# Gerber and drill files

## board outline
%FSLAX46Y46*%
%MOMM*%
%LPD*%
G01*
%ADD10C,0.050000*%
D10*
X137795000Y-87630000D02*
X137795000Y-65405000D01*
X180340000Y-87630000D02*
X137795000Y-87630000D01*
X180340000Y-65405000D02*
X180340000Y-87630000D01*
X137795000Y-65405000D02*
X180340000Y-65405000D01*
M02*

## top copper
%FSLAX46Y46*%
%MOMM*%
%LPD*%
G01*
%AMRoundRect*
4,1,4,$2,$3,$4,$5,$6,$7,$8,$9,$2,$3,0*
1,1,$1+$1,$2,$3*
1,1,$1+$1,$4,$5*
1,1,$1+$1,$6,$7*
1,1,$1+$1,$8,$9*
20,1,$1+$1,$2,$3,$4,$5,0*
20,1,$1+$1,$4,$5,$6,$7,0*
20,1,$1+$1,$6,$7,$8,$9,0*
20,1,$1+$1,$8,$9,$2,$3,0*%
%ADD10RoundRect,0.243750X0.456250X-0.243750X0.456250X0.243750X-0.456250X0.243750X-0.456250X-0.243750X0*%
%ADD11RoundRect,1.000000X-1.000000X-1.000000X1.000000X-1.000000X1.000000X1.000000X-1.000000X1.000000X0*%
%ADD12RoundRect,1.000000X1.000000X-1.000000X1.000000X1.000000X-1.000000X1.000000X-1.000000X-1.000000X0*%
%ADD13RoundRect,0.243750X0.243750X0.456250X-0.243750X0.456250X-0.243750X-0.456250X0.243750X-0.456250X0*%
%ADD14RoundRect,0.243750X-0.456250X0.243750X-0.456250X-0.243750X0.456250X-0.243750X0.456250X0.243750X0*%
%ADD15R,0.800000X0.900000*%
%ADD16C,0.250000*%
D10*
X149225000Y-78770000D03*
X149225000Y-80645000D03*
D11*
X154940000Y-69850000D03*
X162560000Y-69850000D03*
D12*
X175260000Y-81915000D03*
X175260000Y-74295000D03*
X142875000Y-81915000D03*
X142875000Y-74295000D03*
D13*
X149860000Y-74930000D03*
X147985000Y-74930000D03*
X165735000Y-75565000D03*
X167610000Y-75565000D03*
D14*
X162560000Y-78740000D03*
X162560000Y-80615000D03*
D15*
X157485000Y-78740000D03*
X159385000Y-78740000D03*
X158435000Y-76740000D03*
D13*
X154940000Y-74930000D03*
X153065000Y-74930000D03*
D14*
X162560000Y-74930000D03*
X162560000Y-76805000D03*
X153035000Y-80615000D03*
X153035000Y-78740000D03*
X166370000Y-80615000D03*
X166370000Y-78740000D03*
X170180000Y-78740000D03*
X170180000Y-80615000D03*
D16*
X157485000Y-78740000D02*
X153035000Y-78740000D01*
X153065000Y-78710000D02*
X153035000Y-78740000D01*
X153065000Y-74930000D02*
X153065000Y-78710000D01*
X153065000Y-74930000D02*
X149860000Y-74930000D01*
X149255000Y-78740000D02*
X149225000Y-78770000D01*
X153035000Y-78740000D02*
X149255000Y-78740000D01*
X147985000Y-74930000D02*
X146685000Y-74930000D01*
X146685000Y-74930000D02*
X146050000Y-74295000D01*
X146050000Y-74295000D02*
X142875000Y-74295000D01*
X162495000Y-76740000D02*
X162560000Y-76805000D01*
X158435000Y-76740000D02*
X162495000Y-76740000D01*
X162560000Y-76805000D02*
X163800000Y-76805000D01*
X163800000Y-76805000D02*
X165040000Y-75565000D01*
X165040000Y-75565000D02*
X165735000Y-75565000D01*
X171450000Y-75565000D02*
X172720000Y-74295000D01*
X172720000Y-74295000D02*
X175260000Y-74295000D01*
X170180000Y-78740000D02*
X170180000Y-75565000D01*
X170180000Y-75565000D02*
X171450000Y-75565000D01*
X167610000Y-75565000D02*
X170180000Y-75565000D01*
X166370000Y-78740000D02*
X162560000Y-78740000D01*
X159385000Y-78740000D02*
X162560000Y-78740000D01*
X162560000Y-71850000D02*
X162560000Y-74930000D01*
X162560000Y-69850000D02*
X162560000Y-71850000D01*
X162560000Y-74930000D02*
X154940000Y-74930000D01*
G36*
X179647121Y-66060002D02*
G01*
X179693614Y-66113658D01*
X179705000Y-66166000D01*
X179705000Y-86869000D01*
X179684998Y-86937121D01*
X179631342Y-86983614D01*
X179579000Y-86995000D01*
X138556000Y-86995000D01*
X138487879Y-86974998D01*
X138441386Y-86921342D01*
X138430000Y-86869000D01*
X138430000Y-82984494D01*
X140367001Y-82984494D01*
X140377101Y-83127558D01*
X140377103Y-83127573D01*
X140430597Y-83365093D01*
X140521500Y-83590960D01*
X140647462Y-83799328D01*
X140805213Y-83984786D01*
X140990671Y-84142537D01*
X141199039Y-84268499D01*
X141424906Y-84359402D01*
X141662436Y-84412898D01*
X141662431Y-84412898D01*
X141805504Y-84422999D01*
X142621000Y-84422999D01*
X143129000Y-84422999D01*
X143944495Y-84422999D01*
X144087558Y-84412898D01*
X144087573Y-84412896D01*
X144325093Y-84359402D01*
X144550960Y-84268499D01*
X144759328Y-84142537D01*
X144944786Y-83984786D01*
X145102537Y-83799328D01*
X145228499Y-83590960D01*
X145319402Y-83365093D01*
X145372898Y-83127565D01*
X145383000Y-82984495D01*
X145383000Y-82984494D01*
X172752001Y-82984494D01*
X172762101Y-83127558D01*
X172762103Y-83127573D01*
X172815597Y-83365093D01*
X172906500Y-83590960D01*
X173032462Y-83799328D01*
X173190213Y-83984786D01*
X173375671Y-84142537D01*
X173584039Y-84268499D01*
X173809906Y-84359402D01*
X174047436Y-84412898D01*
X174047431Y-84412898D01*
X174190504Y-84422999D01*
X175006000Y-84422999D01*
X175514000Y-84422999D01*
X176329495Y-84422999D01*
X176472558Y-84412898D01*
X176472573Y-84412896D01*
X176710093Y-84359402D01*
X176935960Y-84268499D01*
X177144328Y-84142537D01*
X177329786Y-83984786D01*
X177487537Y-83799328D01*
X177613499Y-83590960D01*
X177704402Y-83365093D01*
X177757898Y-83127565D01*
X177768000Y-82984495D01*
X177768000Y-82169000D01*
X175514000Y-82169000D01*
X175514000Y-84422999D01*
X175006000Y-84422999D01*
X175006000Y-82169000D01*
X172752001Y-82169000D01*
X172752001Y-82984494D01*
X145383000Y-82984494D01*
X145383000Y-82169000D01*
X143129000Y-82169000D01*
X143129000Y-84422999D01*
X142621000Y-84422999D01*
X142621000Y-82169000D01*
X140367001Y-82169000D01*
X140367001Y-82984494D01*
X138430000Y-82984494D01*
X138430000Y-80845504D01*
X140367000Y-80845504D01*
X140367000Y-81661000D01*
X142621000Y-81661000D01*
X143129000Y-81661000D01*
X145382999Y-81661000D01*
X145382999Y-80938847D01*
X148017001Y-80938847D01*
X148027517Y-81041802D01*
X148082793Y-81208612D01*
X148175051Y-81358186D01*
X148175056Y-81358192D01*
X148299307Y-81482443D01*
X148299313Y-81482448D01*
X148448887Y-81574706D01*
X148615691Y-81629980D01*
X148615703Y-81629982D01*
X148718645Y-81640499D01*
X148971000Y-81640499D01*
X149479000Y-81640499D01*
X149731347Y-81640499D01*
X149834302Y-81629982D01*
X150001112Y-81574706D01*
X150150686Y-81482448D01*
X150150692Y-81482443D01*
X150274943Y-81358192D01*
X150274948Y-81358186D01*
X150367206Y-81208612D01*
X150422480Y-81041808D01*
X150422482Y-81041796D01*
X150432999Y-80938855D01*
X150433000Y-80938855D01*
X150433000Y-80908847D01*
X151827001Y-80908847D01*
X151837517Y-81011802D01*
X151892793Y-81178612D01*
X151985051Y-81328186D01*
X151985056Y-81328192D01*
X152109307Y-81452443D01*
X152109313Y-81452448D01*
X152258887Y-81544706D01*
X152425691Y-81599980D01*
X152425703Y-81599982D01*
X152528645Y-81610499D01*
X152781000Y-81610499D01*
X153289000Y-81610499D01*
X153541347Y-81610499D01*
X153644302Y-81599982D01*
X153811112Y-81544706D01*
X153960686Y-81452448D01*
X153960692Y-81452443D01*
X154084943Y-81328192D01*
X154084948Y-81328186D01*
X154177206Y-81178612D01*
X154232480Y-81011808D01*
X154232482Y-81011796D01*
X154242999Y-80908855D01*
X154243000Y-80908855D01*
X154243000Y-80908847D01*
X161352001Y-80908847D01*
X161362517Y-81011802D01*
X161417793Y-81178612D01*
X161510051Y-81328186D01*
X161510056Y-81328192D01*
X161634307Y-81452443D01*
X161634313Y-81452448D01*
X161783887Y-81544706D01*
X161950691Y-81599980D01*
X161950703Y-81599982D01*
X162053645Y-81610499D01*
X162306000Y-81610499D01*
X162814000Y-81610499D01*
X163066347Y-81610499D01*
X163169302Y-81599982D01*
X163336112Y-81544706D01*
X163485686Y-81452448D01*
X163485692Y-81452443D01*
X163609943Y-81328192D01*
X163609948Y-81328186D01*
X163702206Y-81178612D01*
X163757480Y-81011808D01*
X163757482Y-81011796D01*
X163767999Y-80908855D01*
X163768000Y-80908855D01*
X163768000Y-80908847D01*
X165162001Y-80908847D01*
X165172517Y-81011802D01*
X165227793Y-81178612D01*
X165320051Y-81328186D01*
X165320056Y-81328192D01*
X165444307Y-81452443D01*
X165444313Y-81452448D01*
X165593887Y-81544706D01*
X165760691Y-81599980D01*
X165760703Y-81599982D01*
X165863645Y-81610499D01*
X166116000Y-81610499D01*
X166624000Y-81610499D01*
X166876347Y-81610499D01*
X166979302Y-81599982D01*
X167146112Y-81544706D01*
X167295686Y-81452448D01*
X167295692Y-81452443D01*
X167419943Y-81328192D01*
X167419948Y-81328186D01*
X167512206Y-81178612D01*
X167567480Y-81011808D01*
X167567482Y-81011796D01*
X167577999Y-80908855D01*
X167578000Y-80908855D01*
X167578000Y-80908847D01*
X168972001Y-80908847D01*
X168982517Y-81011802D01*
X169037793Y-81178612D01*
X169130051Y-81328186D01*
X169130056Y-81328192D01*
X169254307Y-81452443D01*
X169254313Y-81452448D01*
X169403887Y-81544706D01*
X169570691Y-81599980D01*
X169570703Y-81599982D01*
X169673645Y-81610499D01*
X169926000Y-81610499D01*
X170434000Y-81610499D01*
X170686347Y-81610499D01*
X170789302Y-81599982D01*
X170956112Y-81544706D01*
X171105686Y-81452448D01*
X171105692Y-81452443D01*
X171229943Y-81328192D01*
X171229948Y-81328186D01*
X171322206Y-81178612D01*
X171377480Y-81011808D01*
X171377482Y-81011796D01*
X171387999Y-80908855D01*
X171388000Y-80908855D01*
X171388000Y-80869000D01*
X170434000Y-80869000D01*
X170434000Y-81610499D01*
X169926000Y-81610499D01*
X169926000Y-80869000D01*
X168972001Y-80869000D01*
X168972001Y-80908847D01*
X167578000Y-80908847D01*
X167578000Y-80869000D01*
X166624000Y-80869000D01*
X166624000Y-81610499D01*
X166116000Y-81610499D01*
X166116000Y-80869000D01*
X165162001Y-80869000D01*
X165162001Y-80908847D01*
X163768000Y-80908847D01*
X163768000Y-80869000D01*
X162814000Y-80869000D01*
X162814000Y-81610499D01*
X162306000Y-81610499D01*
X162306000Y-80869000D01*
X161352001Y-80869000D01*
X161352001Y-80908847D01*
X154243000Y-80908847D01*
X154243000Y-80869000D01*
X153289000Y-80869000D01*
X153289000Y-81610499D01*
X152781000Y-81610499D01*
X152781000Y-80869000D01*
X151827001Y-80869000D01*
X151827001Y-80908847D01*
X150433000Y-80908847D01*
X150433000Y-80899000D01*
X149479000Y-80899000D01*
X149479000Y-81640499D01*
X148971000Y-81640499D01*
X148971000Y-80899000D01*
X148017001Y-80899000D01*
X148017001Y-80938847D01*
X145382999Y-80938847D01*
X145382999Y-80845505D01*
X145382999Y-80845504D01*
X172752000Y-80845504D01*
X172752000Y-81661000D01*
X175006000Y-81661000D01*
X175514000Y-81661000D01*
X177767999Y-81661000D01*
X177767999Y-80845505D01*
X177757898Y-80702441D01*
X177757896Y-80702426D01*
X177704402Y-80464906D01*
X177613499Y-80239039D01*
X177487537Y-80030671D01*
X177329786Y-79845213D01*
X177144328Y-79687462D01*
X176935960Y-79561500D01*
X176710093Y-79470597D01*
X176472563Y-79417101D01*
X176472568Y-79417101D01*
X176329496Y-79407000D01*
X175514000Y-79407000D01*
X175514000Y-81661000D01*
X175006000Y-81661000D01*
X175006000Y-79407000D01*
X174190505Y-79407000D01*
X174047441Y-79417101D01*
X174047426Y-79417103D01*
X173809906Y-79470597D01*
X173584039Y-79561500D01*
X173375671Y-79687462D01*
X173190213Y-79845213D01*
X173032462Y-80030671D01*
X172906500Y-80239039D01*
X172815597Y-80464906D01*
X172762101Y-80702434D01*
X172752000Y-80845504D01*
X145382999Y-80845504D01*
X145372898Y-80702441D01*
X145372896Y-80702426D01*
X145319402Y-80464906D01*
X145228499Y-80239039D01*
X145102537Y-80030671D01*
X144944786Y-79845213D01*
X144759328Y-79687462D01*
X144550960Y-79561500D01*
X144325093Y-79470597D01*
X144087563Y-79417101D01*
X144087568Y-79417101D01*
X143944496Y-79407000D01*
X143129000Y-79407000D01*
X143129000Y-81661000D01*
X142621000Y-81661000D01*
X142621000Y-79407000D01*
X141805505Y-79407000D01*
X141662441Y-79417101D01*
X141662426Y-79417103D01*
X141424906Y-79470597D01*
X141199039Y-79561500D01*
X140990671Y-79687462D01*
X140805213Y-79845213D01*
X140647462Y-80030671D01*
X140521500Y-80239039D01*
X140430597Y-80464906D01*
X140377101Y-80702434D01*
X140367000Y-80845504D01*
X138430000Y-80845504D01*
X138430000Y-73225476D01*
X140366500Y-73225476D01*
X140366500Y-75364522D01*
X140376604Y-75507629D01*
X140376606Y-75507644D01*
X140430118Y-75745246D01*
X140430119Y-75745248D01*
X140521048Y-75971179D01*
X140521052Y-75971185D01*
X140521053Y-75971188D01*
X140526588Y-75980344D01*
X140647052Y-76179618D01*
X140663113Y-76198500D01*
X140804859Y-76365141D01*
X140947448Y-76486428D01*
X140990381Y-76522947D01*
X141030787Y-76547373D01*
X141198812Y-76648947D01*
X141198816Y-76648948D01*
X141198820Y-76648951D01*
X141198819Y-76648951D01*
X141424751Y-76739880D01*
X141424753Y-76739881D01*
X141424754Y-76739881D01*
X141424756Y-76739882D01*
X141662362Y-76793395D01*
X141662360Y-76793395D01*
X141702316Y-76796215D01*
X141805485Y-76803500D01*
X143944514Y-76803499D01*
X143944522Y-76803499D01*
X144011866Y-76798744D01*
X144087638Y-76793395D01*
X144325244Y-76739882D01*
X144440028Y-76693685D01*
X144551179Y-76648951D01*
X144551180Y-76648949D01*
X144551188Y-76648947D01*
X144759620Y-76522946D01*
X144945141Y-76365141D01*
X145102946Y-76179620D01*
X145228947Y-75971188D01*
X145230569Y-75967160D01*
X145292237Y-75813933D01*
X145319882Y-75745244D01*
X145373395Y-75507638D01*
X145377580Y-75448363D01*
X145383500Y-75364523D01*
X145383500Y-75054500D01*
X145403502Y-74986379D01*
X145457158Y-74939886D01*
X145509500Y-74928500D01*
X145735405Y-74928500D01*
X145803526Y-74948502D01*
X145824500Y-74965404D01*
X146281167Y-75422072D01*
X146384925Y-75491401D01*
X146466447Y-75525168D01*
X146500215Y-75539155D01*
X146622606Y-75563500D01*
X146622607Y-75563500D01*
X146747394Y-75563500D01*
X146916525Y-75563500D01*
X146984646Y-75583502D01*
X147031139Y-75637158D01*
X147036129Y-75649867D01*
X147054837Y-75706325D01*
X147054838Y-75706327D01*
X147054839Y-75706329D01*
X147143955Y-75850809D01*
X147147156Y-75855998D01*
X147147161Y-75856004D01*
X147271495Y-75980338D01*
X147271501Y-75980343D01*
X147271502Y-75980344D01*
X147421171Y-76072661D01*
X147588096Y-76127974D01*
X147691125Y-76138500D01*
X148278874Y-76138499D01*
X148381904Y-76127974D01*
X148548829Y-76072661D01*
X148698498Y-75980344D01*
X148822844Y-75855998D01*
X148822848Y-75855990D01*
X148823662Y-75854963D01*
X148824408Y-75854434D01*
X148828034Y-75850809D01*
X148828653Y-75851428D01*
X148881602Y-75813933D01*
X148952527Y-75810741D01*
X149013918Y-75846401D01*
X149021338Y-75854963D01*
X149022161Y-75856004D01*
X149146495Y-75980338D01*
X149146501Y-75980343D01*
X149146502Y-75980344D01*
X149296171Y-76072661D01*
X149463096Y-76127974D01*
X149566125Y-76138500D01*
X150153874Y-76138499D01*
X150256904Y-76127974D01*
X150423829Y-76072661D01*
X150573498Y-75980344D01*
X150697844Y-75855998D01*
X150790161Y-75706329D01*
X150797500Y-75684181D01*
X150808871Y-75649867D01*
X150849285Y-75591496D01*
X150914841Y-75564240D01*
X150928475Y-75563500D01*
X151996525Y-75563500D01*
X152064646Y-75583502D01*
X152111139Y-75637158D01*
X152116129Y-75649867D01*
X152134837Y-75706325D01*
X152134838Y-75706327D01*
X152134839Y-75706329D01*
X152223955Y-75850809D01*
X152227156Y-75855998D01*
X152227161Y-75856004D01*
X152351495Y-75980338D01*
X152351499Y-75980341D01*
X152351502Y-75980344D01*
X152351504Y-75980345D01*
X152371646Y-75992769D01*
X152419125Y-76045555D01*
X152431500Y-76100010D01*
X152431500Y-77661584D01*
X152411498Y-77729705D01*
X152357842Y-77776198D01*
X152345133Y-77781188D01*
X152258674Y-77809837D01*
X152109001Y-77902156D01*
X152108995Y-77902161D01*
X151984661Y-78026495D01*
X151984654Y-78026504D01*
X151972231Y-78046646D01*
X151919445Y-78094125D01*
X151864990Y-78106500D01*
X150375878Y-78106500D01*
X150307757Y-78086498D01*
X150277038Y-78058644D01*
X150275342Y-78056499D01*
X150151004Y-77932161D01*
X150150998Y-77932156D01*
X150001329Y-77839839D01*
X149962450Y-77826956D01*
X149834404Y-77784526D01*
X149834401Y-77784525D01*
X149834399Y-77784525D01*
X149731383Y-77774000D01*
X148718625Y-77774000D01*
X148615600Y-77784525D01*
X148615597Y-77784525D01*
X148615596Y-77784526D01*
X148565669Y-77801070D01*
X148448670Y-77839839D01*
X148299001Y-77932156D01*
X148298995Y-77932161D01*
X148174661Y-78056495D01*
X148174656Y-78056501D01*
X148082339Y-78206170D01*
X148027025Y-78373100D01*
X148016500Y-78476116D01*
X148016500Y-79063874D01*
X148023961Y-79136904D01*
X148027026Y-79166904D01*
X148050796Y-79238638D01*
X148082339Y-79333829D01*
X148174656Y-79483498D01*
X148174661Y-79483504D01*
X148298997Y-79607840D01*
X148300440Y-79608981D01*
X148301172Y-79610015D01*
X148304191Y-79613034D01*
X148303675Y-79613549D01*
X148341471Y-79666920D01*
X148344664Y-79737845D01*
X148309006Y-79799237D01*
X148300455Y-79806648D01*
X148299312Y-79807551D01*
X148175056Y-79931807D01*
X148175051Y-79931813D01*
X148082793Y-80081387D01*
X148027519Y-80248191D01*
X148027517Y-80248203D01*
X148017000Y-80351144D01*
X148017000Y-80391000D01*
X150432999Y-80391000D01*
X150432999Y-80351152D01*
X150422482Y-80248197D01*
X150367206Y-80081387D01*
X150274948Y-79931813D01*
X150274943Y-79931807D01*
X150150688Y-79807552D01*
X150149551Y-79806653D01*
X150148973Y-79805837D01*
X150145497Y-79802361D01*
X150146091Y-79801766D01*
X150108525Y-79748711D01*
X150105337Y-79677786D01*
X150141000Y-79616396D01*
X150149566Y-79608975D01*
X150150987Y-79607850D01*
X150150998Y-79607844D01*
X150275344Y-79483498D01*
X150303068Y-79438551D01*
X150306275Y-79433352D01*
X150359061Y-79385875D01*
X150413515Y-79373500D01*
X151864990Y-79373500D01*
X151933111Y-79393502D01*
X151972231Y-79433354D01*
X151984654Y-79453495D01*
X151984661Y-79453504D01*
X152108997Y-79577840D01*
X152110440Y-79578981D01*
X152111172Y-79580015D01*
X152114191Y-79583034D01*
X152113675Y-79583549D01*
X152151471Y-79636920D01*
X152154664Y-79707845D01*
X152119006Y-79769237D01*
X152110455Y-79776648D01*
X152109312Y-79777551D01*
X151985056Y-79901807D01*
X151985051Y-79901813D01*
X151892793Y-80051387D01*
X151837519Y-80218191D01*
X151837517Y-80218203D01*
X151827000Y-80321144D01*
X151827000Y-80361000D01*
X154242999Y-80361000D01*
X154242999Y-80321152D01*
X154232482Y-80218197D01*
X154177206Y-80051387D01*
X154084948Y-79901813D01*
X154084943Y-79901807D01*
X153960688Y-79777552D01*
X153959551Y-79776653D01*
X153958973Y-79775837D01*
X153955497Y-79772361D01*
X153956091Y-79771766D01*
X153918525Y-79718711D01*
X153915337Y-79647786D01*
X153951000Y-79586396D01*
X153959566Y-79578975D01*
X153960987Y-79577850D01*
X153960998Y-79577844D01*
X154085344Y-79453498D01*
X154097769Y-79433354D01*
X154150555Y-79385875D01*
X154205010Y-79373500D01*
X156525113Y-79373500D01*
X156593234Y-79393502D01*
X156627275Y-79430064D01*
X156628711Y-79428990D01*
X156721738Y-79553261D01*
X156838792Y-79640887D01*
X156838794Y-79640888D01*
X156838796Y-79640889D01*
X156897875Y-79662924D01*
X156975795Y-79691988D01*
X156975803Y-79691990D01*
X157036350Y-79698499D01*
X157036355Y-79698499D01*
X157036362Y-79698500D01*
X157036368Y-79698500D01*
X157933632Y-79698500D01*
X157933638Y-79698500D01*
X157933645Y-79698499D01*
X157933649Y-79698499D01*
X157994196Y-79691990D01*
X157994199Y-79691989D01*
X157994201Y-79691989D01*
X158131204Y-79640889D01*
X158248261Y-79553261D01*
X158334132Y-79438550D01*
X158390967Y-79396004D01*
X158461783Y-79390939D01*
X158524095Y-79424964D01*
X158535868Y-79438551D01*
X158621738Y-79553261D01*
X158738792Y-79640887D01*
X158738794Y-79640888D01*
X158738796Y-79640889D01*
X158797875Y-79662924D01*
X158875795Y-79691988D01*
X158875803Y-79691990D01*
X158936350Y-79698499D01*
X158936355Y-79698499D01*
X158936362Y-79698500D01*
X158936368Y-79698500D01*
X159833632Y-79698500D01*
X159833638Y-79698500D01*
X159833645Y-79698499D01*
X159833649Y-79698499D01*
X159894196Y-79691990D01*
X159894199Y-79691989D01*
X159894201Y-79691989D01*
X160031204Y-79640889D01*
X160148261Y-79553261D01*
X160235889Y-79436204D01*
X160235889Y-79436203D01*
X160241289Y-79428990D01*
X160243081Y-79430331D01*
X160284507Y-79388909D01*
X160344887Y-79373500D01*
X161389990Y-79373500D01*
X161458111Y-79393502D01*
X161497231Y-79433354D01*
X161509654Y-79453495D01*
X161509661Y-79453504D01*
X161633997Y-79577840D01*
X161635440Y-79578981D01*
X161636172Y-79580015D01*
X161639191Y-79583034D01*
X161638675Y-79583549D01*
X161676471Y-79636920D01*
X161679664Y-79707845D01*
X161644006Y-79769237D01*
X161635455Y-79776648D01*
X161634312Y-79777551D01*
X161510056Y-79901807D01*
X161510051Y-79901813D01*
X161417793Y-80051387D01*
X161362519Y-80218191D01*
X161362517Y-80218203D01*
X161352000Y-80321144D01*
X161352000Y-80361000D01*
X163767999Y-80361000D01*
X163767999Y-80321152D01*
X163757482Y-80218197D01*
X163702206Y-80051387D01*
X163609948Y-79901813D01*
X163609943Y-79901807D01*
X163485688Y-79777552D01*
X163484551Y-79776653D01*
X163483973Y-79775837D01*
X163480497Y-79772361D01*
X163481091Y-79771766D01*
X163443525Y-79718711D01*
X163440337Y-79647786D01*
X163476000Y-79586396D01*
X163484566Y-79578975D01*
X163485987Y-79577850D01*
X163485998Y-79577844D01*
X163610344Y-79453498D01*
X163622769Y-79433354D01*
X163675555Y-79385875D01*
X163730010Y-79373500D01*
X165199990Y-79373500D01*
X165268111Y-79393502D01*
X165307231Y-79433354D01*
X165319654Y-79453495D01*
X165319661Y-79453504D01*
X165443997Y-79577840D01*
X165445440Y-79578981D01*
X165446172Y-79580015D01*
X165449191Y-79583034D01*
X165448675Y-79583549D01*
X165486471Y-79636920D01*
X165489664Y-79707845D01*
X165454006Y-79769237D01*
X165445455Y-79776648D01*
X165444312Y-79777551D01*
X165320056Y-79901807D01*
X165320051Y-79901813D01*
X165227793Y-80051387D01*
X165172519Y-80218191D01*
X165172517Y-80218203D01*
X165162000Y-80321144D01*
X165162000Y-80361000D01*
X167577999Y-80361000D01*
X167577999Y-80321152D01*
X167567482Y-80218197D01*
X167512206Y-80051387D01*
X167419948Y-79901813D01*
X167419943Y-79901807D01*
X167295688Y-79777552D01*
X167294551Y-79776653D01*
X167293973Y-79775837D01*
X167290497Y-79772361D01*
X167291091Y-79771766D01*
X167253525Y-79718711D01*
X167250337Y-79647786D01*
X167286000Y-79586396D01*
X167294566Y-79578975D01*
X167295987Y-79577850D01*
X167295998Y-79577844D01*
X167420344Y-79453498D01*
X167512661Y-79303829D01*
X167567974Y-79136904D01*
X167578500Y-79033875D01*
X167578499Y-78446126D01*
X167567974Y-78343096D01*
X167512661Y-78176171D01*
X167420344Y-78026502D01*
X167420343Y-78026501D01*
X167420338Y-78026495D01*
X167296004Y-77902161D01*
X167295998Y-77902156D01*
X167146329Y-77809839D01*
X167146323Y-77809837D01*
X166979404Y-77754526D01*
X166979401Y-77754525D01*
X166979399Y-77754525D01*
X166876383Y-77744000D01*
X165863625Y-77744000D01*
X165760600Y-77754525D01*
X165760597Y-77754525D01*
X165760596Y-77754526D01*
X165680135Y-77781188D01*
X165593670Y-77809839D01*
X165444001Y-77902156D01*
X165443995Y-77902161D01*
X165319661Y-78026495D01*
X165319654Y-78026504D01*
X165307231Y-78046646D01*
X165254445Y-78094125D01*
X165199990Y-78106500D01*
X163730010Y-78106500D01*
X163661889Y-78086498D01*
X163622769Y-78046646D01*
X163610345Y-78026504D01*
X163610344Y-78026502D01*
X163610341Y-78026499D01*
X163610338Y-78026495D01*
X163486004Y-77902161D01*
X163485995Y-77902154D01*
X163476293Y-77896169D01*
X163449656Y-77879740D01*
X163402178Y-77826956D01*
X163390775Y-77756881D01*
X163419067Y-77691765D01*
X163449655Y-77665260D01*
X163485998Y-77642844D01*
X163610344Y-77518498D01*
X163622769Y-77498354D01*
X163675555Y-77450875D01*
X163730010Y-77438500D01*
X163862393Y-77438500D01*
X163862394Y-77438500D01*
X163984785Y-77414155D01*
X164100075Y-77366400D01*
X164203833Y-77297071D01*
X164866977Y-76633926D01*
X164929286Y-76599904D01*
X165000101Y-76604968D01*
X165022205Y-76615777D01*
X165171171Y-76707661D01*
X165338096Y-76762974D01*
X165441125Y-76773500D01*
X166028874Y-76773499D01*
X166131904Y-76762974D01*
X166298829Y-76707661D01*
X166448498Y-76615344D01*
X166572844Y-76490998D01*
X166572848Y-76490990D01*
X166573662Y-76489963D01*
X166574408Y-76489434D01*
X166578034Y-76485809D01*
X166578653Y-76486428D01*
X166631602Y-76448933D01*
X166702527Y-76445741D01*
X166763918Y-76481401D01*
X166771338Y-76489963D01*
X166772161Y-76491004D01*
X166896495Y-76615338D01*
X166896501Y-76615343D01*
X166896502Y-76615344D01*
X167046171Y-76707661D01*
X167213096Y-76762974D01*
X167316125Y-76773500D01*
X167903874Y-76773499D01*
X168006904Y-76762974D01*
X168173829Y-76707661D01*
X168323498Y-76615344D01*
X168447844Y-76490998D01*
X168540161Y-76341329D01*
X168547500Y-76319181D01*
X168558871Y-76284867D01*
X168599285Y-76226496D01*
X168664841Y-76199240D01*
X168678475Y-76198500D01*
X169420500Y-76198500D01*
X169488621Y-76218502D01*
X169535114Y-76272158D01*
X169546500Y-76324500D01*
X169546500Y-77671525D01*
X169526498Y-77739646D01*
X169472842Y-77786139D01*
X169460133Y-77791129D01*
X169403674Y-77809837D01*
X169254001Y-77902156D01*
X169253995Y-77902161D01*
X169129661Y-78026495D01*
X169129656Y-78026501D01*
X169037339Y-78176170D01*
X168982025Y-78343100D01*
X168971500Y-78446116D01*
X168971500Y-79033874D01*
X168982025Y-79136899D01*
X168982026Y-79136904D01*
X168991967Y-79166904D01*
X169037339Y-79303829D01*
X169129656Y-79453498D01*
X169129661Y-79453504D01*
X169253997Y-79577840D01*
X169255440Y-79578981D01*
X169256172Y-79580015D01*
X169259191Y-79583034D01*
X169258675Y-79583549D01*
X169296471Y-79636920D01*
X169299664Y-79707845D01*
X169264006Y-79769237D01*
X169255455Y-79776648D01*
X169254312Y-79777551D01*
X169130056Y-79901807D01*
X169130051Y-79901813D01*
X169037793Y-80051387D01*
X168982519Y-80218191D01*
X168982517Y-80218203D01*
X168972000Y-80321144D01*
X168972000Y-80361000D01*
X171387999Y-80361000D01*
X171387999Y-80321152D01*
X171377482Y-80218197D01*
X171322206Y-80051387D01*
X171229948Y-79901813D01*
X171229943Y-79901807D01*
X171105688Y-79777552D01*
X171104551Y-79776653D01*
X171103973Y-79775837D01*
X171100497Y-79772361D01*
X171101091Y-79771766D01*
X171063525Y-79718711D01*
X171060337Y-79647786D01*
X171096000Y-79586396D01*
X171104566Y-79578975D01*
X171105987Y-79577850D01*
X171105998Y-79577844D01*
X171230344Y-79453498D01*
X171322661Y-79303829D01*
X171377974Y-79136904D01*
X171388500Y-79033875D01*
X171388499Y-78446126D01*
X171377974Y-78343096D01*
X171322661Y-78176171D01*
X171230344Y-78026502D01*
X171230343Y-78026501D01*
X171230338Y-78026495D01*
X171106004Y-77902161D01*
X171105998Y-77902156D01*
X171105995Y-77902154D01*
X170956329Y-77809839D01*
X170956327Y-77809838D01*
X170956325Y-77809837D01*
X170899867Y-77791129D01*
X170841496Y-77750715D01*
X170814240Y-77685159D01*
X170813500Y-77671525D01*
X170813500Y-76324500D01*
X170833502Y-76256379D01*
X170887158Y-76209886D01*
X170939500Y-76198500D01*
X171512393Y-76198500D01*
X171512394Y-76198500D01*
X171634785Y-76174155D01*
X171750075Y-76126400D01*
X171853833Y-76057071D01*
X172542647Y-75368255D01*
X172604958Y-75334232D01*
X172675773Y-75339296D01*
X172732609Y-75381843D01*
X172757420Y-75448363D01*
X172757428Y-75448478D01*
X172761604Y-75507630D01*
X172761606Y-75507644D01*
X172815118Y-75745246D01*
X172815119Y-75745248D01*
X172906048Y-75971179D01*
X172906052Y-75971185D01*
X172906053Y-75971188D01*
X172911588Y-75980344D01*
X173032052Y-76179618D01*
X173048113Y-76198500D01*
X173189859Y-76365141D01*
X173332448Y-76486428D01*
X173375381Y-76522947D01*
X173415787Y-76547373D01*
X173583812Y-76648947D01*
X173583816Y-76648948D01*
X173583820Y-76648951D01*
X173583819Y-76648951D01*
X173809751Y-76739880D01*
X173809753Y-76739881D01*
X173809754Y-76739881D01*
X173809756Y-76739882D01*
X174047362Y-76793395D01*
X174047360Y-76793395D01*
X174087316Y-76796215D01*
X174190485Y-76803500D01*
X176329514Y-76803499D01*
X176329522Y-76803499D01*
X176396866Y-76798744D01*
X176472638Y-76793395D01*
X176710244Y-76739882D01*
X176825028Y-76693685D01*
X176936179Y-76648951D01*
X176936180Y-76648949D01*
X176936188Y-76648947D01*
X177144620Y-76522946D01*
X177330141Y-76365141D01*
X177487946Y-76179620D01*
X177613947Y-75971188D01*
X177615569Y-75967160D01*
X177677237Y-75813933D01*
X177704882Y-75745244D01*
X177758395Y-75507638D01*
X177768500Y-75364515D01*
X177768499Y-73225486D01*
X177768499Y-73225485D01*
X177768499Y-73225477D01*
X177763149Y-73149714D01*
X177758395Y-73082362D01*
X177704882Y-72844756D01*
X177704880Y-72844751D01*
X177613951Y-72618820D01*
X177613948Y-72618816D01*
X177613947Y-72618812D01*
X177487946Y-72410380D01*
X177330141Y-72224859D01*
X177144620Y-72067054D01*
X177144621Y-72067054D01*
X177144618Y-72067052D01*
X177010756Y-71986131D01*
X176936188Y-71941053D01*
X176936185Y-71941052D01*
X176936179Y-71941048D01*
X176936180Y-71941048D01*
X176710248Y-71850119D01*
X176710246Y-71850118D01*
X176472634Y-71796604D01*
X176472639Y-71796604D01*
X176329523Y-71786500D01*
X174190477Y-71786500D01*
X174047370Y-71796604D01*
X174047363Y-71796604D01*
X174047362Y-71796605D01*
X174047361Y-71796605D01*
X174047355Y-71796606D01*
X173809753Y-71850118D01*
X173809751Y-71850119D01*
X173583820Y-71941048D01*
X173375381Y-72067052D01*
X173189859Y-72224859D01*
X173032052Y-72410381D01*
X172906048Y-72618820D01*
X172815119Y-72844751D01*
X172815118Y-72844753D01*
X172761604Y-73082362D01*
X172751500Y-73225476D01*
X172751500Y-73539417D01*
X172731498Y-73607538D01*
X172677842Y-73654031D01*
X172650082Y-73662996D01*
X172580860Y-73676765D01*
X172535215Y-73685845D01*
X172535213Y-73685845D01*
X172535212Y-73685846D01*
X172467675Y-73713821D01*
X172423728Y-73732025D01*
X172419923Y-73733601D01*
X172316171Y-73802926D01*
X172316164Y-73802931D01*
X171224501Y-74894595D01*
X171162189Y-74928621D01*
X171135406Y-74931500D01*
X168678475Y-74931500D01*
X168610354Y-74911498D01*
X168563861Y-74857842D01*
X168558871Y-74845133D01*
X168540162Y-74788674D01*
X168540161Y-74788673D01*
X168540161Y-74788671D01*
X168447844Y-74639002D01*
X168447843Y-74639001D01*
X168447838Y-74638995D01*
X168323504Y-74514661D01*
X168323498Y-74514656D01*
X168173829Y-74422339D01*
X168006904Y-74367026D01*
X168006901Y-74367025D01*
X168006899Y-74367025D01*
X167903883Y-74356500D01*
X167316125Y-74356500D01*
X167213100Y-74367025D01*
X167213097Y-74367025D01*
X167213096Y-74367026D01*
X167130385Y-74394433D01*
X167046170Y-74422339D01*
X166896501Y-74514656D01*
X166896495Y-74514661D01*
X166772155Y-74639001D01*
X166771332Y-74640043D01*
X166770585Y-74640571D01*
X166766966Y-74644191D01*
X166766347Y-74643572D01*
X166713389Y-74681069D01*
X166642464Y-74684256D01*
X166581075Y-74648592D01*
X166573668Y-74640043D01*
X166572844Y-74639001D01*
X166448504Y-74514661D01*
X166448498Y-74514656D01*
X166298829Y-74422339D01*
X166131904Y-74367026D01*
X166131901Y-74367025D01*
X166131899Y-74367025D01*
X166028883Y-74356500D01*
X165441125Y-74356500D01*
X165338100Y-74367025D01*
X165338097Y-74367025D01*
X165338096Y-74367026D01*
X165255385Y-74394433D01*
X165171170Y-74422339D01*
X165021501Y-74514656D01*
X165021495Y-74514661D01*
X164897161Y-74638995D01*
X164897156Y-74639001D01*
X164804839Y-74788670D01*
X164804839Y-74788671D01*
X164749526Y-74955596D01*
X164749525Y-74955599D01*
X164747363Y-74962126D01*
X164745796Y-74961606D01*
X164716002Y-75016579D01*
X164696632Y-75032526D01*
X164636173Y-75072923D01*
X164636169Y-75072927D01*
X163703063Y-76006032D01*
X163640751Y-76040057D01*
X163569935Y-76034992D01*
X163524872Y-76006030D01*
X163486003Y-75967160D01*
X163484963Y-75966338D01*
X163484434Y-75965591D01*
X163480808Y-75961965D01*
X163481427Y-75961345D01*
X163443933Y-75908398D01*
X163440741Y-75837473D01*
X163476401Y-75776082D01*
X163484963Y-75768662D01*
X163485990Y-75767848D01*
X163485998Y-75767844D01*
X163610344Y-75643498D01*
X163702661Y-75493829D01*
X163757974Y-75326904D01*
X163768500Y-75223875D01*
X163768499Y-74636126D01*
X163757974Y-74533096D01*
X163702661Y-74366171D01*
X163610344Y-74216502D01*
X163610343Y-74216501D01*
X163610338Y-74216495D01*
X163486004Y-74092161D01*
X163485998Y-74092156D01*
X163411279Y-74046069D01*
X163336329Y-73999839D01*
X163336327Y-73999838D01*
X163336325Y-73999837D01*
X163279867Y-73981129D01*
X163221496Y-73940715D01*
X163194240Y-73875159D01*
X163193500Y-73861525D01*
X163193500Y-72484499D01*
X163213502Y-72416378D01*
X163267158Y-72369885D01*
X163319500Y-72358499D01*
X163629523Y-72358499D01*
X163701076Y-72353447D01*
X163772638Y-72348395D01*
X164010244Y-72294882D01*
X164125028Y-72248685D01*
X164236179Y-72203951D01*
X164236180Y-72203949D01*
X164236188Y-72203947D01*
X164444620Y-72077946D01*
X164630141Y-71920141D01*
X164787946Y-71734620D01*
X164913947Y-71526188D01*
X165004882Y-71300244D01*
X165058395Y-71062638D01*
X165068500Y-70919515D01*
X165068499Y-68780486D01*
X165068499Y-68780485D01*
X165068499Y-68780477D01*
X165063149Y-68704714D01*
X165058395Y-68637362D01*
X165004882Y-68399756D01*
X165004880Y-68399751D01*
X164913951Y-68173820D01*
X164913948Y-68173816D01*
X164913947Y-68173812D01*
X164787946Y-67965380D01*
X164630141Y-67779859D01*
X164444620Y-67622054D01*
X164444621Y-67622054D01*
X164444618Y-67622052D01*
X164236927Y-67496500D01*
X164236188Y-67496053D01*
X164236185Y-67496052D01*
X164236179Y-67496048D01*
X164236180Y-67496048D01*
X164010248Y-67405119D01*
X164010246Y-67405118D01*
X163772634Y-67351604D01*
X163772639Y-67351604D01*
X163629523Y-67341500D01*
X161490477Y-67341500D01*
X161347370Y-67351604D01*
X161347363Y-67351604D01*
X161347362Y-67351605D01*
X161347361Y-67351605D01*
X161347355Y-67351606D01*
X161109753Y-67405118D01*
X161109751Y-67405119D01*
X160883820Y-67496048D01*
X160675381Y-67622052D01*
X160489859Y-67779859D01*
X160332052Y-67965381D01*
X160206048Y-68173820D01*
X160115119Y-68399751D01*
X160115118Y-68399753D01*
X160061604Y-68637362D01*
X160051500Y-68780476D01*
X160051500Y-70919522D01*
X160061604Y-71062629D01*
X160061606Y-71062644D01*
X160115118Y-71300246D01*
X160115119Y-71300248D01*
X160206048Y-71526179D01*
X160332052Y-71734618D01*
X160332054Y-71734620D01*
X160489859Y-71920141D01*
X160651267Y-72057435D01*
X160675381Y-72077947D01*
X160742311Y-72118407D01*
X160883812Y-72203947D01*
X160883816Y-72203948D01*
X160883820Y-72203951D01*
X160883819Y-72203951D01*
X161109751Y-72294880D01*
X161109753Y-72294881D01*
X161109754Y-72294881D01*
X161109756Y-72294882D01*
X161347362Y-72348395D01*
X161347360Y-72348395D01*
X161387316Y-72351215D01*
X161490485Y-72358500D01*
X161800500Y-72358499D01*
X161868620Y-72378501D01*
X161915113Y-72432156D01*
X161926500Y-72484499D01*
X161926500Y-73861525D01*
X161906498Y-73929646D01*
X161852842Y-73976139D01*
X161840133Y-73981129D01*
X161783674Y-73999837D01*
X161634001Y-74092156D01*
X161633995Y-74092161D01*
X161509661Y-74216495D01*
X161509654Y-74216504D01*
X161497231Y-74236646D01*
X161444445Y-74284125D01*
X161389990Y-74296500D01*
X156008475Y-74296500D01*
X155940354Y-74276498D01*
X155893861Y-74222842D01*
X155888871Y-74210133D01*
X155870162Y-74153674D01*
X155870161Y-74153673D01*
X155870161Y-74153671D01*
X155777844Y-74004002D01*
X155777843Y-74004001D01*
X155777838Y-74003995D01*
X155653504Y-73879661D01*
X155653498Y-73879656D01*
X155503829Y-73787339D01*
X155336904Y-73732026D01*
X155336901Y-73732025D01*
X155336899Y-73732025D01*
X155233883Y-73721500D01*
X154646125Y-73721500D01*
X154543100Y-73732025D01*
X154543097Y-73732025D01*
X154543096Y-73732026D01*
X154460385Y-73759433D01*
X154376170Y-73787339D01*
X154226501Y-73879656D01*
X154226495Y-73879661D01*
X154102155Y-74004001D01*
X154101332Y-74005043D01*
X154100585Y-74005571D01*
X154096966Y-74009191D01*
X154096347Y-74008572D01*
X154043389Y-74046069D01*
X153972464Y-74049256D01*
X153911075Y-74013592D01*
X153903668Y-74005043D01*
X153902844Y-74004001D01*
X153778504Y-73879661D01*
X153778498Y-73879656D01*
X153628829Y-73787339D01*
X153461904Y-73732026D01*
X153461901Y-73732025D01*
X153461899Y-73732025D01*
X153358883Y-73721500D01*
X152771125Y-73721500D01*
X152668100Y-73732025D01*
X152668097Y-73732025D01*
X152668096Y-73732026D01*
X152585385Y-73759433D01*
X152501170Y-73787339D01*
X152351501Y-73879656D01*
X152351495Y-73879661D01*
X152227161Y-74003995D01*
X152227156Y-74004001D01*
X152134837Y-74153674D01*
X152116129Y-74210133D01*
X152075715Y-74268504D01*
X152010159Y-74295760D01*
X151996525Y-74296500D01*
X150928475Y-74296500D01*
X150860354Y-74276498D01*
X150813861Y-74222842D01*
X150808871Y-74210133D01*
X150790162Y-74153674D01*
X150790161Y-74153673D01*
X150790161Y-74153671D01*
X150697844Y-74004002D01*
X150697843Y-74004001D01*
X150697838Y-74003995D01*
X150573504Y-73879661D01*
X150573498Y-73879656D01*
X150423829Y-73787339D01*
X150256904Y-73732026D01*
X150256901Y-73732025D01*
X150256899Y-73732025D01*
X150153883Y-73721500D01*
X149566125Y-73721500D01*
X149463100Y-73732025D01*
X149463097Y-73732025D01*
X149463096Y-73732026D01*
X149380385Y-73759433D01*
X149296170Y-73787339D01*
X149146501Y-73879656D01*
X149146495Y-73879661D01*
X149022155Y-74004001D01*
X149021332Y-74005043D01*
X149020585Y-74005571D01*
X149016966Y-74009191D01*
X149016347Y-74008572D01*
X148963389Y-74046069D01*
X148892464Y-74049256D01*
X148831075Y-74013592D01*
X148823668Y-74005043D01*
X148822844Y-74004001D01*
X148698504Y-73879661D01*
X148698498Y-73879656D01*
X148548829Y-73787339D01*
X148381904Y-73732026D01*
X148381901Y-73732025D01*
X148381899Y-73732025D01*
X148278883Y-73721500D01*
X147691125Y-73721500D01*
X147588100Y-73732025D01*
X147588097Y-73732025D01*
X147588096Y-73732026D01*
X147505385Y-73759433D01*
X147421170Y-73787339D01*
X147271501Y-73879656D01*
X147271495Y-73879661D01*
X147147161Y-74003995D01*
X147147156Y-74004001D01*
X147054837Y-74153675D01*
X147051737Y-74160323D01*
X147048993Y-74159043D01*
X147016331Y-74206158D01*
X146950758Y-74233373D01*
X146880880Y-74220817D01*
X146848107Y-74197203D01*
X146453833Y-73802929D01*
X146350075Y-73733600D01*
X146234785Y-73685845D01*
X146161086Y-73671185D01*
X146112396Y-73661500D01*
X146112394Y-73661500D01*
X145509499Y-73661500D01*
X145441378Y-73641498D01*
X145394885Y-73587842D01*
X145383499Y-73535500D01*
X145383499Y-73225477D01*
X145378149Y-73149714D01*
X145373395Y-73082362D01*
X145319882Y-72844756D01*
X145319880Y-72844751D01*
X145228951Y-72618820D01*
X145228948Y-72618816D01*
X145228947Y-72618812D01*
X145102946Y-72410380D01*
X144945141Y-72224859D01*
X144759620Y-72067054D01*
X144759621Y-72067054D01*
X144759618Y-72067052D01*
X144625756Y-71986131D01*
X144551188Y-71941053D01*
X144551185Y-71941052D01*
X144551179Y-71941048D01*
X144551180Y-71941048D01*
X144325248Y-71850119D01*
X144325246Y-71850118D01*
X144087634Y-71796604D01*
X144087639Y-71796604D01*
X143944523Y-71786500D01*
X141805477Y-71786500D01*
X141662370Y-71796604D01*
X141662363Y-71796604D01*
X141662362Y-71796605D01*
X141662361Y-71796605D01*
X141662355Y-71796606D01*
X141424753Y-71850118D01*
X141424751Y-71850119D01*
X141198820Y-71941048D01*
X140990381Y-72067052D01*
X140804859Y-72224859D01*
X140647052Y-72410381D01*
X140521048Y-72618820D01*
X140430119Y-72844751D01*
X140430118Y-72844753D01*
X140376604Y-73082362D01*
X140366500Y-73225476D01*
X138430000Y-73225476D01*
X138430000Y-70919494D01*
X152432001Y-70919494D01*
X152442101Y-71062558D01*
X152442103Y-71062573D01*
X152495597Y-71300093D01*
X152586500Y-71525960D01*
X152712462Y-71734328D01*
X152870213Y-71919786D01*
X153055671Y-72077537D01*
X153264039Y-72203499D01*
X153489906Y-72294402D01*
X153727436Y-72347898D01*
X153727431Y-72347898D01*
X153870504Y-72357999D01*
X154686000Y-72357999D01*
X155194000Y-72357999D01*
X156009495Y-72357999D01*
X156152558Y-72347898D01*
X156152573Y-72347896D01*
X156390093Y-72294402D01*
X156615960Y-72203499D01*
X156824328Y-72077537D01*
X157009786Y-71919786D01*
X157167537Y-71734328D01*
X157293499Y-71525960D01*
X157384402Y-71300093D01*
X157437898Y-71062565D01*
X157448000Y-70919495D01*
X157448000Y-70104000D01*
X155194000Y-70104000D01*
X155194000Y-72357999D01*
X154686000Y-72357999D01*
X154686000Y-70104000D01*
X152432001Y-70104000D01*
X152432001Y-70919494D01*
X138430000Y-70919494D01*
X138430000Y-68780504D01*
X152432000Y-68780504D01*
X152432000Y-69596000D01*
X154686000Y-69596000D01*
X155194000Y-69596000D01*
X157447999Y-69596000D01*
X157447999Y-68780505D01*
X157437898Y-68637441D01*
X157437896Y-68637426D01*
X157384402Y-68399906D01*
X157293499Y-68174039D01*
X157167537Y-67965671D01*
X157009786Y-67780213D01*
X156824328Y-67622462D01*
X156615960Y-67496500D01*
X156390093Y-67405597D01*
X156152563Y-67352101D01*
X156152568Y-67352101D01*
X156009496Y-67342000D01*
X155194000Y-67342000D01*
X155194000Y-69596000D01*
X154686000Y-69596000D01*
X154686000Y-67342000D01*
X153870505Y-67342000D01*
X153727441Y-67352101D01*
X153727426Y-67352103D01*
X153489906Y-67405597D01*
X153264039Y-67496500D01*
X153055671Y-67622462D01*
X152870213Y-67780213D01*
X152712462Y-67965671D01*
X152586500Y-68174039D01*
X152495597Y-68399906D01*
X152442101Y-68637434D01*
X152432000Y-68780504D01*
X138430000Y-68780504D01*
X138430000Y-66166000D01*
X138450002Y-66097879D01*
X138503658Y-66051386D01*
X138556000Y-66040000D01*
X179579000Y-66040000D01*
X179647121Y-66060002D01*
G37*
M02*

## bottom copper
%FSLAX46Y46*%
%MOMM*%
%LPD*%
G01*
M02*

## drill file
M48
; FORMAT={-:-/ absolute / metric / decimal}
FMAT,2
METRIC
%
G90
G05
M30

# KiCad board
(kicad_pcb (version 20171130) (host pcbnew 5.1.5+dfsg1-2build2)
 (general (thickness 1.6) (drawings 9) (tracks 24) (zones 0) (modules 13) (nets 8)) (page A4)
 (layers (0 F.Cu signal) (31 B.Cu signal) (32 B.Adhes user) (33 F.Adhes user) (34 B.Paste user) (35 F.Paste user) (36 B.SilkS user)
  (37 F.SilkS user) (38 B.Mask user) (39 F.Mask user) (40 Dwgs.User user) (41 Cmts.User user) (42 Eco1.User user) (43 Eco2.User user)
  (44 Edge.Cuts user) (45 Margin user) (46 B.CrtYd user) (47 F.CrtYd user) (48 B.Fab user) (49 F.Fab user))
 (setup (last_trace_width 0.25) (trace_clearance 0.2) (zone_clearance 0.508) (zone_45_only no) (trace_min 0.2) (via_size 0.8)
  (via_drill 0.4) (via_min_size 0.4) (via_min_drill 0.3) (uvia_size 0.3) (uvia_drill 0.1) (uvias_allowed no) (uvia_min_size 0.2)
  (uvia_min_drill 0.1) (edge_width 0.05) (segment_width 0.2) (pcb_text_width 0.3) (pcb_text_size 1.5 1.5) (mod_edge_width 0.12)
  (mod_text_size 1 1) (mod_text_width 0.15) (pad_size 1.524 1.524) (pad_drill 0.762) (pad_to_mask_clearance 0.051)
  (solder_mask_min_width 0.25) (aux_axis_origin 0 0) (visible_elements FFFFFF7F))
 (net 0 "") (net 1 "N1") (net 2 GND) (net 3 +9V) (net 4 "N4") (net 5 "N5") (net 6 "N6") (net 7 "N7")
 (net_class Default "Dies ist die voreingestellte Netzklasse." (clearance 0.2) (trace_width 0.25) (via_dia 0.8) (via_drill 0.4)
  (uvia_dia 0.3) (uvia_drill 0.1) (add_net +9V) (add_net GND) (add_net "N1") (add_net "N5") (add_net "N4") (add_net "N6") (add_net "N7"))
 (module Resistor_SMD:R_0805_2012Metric (layer F.Cu) (at 149.225 79.7075 90)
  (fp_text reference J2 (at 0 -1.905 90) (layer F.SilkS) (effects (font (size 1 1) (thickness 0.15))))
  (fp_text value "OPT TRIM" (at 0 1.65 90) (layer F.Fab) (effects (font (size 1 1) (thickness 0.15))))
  (pad 2 smd roundrect (at 0.9375 0 90) (size 0.975 1.4) (layers F.Cu F.Paste F.Mask) (roundrect_rratio 0.25) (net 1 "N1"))
  (pad 1 smd roundrect (at -0.9375 0 90) (size 0.975 1.4) (layers F.Cu F.Paste F.Mask) (roundrect_rratio 0.25) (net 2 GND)))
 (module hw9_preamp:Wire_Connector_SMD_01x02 (layer F.Cu) (at 158.75 69.85)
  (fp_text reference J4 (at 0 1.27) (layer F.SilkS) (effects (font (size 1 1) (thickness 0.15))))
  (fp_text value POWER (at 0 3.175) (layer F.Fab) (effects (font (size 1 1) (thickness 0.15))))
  (pad 1 smd roundrect (at -3.81 0) (size 4 4) (layers F.Cu F.Paste F.Mask) (roundrect_rratio 0.25) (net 2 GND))
  (pad 2 smd roundrect (at 3.81 0) (size 4 4) (layers F.Cu F.Paste F.Mask) (roundrect_rratio 0.25) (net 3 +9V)))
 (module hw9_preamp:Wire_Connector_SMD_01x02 (layer F.Cu) (at 175.26 78.105 90)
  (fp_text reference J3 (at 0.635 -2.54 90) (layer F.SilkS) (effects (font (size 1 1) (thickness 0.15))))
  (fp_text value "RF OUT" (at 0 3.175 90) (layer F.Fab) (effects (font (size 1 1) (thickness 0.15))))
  (pad 1 smd roundrect (at -3.81 0 90) (size 4 4) (layers F.Cu F.Paste F.Mask) (roundrect_rratio 0.25) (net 2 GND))
  (pad 2 smd roundrect (at 3.81 0 90) (size 4 4) (layers F.Cu F.Paste F.Mask) (roundrect_rratio 0.25) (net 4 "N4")))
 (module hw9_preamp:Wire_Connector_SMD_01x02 (layer F.Cu) (at 142.875 78.105 90)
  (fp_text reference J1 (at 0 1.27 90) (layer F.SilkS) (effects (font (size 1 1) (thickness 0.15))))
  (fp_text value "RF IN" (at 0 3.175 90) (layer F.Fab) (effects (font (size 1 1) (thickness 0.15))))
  (pad 1 smd roundrect (at -3.81 0 90) (size 4 4) (layers F.Cu F.Paste F.Mask) (roundrect_rratio 0.25) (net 2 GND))
  (pad 2 smd roundrect (at 3.81 0 90) (size 4 4) (layers F.Cu F.Paste F.Mask) (roundrect_rratio 0.25) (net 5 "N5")))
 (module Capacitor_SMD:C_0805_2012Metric (layer F.Cu) (at 148.9225 74.93 180)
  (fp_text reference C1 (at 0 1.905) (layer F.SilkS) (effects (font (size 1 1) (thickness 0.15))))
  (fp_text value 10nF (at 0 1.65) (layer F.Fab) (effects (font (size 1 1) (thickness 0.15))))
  (pad 1 smd roundrect (at -0.9375 0 180) (size 0.975 1.4) (layers F.Cu F.Paste F.Mask) (roundrect_rratio 0.25) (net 1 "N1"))
  (pad 2 smd roundrect (at 0.9375 0 180) (size 0.975 1.4) (layers F.Cu F.Paste F.Mask) (roundrect_rratio 0.25) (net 5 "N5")))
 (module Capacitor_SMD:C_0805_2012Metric (layer F.Cu) (at 166.6725 75.565 180)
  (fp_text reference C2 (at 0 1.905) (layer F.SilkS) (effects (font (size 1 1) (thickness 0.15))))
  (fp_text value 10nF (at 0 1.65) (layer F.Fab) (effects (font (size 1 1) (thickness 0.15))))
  (pad 2 smd roundrect (at 0.9375 0 180) (size 0.975 1.4) (layers F.Cu F.Paste F.Mask) (roundrect_rratio 0.25) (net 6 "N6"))
  (pad 1 smd roundrect (at -0.9375 0 180) (size 0.975 1.4) (layers F.Cu F.Paste F.Mask) (roundrect_rratio 0.25) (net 4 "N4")))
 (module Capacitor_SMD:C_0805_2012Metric (layer F.Cu) (at 162.56 79.6775 270)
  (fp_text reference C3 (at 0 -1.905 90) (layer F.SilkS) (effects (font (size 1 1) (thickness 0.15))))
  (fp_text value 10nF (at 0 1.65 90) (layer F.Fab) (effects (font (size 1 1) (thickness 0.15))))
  (pad 1 smd roundrect (at -0.9375 0 270) (size 0.975 1.4) (layers F.Cu F.Paste F.Mask) (roundrect_rratio 0.25) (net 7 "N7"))
  (pad 2 smd roundrect (at 0.9375 0 270) (size 0.975 1.4) (layers F.Cu F.Paste F.Mask) (roundrect_rratio 0.25) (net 2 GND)))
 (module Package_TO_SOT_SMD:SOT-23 (layer F.Cu) (at 158.435 77.74 90)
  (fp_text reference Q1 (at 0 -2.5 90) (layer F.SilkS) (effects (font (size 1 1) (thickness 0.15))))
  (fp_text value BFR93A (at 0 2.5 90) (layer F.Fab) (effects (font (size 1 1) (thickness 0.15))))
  (pad 1 smd rect (at -1 -0.95 90) (size 0.9 0.8) (layers F.Cu F.Paste F.Mask) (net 1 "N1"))
  (pad 2 smd rect (at -1 0.95 90) (size 0.9 0.8) (layers F.Cu F.Paste F.Mask) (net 7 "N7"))
  (pad 3 smd rect (at 1 0 90) (size 0.9 0.8) (layers F.Cu F.Paste F.Mask) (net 6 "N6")))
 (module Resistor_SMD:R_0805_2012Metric (layer F.Cu) (at 154.0025 74.93 180)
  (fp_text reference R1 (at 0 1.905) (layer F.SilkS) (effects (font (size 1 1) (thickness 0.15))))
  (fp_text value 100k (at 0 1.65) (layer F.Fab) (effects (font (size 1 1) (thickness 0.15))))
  (pad 1 smd roundrect (at -0.9375 0 180) (size 0.975 1.4) (layers F.Cu F.Paste F.Mask) (roundrect_rratio 0.25) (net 3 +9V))
  (pad 2 smd roundrect (at 0.9375 0 180) (size 0.975 1.4) (layers F.Cu F.Paste F.Mask) (roundrect_rratio 0.25) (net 1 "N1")))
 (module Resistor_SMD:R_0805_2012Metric (layer F.Cu) (at 162.56 75.8675 270)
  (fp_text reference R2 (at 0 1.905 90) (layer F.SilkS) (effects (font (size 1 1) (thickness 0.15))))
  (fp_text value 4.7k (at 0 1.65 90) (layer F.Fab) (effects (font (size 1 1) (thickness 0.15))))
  (pad 1 smd roundrect (at -0.9375 0 270) (size 0.975 1.4) (layers F.Cu F.Paste F.Mask) (roundrect_rratio 0.25) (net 3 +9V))
  (pad 2 smd roundrect (at 0.9375 0 270) (size 0.975 1.4) (layers F.Cu F.Paste F.Mask) (roundrect_rratio 0.25) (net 6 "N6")))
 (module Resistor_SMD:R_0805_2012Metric (layer F.Cu) (at 153.035 79.6775 270)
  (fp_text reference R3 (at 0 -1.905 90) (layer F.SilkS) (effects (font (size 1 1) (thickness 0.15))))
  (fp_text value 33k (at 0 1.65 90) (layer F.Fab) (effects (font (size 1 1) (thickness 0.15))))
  (pad 2 smd roundrect (at 0.9375 0 270) (size 0.975 1.4) (layers F.Cu F.Paste F.Mask) (roundrect_rratio 0.25) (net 2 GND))
  (pad 1 smd roundrect (at -0.9375 0 270) (size 0.975 1.4) (layers F.Cu F.Paste F.Mask) (roundrect_rratio 0.25) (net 1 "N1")))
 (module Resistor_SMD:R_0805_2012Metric (layer F.Cu) (at 166.37 79.6775 270)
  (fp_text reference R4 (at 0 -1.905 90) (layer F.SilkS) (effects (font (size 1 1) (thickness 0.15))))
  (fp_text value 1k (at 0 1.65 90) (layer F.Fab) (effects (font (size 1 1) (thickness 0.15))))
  (pad 2 smd roundrect (at 0.9375 0 270) (size 0.975 1.4) (layers F.Cu F.Paste F.Mask) (roundrect_rratio 0.25) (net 2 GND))
  (pad 1 smd roundrect (at -0.9375 0 270) (size 0.975 1.4) (layers F.Cu F.Paste F.Mask) (roundrect_rratio 0.25) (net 7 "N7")))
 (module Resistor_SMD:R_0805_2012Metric (layer F.Cu) (at 170.18 79.6775 270)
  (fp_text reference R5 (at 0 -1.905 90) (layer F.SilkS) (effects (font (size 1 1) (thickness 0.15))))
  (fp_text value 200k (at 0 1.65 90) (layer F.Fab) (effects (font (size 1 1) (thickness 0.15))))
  (pad 1 smd roundrect (at -0.9375 0 270) (size 0.975 1.4) (layers F.Cu F.Paste F.Mask) (roundrect_rratio 0.25) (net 4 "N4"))
  (pad 2 smd roundrect (at 0.9375 0 270) (size 0.975 1.4) (layers F.Cu F.Paste F.Mask) (roundrect_rratio 0.25) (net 2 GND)))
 (gr_line (start 137.795 87.63) (end 137.795 65.405) (layer Edge.Cuts) (width 0.05))
 (gr_line (start 180.34 87.63) (end 137.795 87.63) (layer Edge.Cuts) (width 0.05))
 (gr_line (start 180.34 65.405) (end 180.34 87.63) (layer Edge.Cuts) (width 0.05))
 (gr_line (start 137.795 65.405) (end 180.34 65.405) (layer Edge.Cuts) (width 0.05))
 (segment (start 157.485 78.74) (end 153.035 78.74) (width 0.25) (layer F.Cu) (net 1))
 (segment (start 153.065 78.71) (end 153.035 78.74) (width 0.25) (layer F.Cu) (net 1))
 (segment (start 153.065 74.93) (end 153.065 78.71) (width 0.25) (layer F.Cu) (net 1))
 (segment (start 153.065 74.93) (end 149.86 74.93) (width 0.25) (layer F.Cu) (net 1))
 (segment (start 149.255 78.74) (end 149.225 78.77) (width 0.25) (layer F.Cu) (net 1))
 (segment (start 153.035 78.74) (end 149.255 78.74) (width 0.25) (layer F.Cu) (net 1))
 (segment (start 147.985 74.93) (end 146.685 74.93) (width 0.25) (layer F.Cu) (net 5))
 (segment (start 146.685 74.93) (end 146.05 74.295) (width 0.25) (layer F.Cu) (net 5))
 (segment (start 146.05 74.295) (end 142.875 74.295) (width 0.25) (layer F.Cu) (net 5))
 (segment (start 162.495 76.74) (end 162.56 76.805) (width 0.25) (layer F.Cu) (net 6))
 (segment (start 158.435 76.74) (end 162.495 76.74) (width 0.25) (layer F.Cu) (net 6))
 (segment (start 162.56 76.805) (end 163.8 76.805) (width 0.25) (layer F.Cu) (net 6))
 (segment (start 163.8 76.805) (end 165.04 75.565) (width 0.25) (layer F.Cu) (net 6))
 (segment (start 165.04 75.565) (end 165.735 75.565) (width 0.25) (layer F.Cu) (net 6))
 (segment (start 171.45 75.565) (end 172.72 74.295) (width 0.25) (layer F.Cu) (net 4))
 (segment (start 172.72 74.295) (end 175.26 74.295) (width 0.25) (layer F.Cu) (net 4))
 (segment (start 170.18 78.74) (end 170.18 75.565) (width 0.25) (layer F.Cu) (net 4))
 (segment (start 170.18 75.565) (end 171.45 75.565) (width 0.25) (layer F.Cu) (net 4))
 (segment (start 167.61 75.565) (end 170.18 75.565) (width 0.25) (layer F.Cu) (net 4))
 (segment (start 166.37 78.74) (end 162.56 78.74) (width 0.25) (layer F.Cu) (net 7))
 (segment (start 159.385 78.74) (end 162.56 78.74) (width 0.25) (layer F.Cu) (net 7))
 (segment (start 162.56 71.85) (end 162.56 74.93) (width 0.25) (layer F.Cu) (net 3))
 (segment (start 162.56 69.85) (end 162.56 71.85) (width 0.25) (layer F.Cu) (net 3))
 (segment (start 162.56 74.93) (end 154.94 74.93) (width 0.25) (layer F.Cu) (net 3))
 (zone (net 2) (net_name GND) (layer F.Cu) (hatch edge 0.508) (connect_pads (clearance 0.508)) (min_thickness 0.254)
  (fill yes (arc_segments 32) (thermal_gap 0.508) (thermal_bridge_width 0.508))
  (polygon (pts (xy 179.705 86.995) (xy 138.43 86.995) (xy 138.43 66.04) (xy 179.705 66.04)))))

